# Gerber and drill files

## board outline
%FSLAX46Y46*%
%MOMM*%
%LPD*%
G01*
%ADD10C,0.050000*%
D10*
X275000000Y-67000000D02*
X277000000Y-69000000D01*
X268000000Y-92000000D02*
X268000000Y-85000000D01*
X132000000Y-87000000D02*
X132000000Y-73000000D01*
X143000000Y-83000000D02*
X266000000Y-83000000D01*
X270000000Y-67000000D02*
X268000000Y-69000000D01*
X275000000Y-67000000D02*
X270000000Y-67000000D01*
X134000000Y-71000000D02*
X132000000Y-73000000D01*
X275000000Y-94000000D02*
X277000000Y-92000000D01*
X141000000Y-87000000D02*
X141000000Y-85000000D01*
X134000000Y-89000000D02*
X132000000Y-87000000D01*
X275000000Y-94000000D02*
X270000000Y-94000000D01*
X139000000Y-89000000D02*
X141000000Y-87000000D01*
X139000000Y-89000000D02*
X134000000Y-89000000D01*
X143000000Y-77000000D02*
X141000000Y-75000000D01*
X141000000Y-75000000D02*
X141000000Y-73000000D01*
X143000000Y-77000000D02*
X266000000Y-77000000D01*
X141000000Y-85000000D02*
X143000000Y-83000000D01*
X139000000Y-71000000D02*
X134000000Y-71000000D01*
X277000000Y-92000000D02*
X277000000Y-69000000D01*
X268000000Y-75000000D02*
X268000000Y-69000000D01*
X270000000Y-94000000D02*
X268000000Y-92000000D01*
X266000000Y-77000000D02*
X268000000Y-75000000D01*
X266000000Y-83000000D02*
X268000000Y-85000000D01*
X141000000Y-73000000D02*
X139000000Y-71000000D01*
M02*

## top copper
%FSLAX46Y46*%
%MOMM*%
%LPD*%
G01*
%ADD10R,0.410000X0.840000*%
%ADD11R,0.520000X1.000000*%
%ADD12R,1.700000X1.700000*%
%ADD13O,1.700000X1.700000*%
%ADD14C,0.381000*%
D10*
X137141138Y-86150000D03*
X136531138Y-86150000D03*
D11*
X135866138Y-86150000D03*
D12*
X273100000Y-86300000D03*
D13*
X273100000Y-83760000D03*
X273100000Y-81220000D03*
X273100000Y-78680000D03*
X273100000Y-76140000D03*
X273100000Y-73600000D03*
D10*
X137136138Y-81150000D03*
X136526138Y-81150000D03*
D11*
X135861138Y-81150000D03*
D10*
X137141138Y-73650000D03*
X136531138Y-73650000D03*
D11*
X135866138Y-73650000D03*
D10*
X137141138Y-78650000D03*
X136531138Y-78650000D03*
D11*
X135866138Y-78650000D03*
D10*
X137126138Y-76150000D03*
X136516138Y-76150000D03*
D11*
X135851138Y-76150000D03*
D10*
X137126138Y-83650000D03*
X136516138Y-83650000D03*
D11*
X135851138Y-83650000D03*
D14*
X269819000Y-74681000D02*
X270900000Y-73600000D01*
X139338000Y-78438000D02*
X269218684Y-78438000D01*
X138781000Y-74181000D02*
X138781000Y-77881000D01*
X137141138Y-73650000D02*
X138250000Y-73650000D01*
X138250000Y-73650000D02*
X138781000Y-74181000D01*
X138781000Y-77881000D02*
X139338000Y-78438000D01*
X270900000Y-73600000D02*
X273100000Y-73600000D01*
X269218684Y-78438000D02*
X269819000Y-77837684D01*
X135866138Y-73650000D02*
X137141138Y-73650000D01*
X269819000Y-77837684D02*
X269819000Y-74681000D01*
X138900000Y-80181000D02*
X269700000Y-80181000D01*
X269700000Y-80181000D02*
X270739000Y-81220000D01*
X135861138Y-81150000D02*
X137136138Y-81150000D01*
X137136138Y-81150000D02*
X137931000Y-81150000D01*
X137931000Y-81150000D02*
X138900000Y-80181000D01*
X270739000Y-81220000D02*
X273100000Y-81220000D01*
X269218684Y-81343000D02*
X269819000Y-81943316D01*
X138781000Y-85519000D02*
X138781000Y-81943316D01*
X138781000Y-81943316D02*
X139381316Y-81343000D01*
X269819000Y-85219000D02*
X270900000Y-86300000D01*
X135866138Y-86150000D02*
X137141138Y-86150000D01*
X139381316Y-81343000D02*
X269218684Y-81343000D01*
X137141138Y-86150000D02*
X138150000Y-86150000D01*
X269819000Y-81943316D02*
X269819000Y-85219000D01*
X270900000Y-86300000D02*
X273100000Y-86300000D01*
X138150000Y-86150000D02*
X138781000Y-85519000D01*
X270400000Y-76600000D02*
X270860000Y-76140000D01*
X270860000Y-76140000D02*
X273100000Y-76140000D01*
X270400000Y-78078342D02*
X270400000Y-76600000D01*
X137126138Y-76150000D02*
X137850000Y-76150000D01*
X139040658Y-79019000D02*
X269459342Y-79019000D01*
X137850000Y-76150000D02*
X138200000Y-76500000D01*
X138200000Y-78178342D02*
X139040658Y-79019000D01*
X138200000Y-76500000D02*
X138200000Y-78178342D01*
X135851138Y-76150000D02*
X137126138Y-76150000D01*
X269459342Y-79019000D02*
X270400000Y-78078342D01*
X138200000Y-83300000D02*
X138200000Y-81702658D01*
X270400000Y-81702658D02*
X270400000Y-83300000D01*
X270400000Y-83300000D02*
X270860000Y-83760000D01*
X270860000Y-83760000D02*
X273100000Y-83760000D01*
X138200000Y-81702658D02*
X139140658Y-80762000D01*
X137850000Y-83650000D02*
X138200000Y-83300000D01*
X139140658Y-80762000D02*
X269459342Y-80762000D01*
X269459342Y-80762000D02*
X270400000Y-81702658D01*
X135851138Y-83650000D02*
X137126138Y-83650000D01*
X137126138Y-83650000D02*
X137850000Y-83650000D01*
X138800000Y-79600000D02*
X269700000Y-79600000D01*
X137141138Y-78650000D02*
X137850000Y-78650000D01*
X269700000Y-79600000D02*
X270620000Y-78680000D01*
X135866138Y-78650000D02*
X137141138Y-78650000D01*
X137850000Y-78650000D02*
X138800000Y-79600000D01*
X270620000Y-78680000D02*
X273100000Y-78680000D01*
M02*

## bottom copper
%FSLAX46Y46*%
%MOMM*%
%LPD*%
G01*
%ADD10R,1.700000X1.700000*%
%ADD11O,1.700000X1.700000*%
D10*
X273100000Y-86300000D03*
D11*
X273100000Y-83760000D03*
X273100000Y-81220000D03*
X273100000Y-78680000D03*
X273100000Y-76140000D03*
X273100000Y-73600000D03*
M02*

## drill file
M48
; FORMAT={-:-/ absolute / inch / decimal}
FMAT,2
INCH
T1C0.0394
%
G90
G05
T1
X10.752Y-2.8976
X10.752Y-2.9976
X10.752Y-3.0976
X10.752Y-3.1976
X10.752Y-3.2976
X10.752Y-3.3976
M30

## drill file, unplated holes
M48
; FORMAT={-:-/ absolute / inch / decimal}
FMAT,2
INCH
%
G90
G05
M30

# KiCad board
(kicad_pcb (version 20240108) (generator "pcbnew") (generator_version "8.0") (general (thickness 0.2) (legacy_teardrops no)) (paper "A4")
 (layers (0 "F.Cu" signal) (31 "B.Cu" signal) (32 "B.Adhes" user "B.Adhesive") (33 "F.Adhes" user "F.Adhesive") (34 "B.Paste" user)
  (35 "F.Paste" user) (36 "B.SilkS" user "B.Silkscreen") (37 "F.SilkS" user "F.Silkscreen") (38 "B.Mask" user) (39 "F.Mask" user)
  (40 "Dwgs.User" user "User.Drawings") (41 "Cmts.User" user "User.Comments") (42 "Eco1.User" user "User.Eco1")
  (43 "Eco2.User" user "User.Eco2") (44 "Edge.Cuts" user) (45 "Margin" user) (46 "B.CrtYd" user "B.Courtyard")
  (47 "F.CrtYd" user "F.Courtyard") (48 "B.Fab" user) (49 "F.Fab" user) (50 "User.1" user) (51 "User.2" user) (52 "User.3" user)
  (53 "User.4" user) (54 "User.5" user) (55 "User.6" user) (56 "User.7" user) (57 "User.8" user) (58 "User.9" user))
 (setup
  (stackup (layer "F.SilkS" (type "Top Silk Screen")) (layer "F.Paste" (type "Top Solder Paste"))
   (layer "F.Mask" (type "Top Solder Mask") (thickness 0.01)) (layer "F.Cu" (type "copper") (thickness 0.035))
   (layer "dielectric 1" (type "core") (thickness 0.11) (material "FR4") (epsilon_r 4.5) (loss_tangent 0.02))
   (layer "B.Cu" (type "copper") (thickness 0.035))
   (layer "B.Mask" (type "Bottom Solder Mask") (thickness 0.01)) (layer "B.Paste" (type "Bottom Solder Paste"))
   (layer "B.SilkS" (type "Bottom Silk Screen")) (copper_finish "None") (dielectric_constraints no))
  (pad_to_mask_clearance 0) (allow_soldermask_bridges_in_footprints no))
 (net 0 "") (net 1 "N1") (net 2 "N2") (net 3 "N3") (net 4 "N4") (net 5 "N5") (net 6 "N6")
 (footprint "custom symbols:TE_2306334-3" (layer "F.Cu") (at 136.446138 86.15 180)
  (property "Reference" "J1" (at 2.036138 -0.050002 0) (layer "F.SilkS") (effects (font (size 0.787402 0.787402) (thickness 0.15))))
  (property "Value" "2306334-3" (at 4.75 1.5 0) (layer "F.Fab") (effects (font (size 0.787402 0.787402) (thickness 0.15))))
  (pad "1_1" smd rect (at -0.695 0 180) (size 0.41 0.84) (layers "F.Cu" "F.Paste" "F.Mask") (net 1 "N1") (solder_mask_margin 0.102))
  (pad "1_2" smd rect (at -0.085 0 180) (size 0.41 0.84) (layers "F.Cu" "F.Paste" "F.Mask") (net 1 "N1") (solder_mask_margin 0.102))
  (pad "1_3" smd rect (at 0.58 0 180) (size 0.52 1) (layers "F.Cu" "F.Paste" "F.Mask") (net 1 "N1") (solder_mask_margin 0.102)))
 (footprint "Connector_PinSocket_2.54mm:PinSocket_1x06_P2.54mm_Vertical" (layer "F.Cu") (at 273.1 86.3 180)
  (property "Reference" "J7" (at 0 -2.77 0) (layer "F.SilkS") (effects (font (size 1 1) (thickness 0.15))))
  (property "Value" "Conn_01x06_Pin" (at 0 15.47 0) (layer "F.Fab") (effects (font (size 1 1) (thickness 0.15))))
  (pad "1" thru_hole rect (at 0 0 180) (size 1.7 1.7) (drill 1) (layers "*.Cu" "*.Mask") (remove_unused_layers no) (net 1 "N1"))
  (pad "2" thru_hole oval (at 0 2.54 180) (size 1.7 1.7) (drill 1) (layers "*.Cu" "*.Mask") (remove_unused_layers no) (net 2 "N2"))
  (pad "3" thru_hole oval (at 0 5.08 180) (size 1.7 1.7) (drill 1) (layers "*.Cu" "*.Mask") (remove_unused_layers no) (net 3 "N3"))
  (pad "4" thru_hole oval (at 0 7.62 180) (size 1.7 1.7) (drill 1) (layers "*.Cu" "*.Mask") (remove_unused_layers no) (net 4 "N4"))
  (pad "5" thru_hole oval (at 0 10.16 180) (size 1.7 1.7) (drill 1) (layers "*.Cu" "*.Mask") (remove_unused_layers no) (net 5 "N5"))
  (pad "6" thru_hole oval (at 0 12.7 180) (size 1.7 1.7) (drill 1) (layers "*.Cu" "*.Mask") (remove_unused_layers no) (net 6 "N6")))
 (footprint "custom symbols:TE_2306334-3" (layer "F.Cu") (at 136.441138 81.15 180)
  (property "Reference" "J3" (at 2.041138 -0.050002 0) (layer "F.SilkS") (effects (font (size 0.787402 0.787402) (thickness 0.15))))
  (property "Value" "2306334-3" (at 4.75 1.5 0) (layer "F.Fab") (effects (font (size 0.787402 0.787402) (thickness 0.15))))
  (pad "1_1" smd rect (at -0.695 0 180) (size 0.41 0.84) (layers "F.Cu" "F.Paste" "F.Mask") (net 3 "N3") (solder_mask_margin 0.102))
  (pad "1_2" smd rect (at -0.085 0 180) (size 0.41 0.84) (layers "F.Cu" "F.Paste" "F.Mask") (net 3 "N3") (solder_mask_margin 0.102))
  (pad "1_3" smd rect (at 0.58 0 180) (size 0.52 1) (layers "F.Cu" "F.Paste" "F.Mask") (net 3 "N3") (solder_mask_margin 0.102)))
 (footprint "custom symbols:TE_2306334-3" (layer "F.Cu") (at 136.446138 73.65 180)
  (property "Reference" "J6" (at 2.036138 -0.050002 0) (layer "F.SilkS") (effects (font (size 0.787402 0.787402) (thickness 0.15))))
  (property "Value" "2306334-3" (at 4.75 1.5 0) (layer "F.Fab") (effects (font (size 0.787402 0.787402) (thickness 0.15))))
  (pad "1_1" smd rect (at -0.695 0 180) (size 0.41 0.84) (layers "F.Cu" "F.Paste" "F.Mask") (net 6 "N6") (solder_mask_margin 0.102))
  (pad "1_2" smd rect (at -0.085 0 180) (size 0.41 0.84) (layers "F.Cu" "F.Paste" "F.Mask") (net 6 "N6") (solder_mask_margin 0.102))
  (pad "1_3" smd rect (at 0.58 0 180) (size 0.52 1) (layers "F.Cu" "F.Paste" "F.Mask") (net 6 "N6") (solder_mask_margin 0.102)))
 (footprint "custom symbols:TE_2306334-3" (layer "F.Cu") (at 136.446138 78.65 180)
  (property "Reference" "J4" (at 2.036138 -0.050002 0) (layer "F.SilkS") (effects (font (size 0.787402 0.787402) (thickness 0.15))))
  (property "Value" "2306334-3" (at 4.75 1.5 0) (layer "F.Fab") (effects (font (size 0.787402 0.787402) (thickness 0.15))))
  (pad "1_1" smd rect (at -0.695 0 180) (size 0.41 0.84) (layers "F.Cu" "F.Paste" "F.Mask") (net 4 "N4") (solder_mask_margin 0.102))
  (pad "1_2" smd rect (at -0.085 0 180) (size 0.41 0.84) (layers "F.Cu" "F.Paste" "F.Mask") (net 4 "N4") (solder_mask_margin 0.102))
  (pad "1_3" smd rect (at 0.58 0 180) (size 0.52 1) (layers "F.Cu" "F.Paste" "F.Mask") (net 4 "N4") (solder_mask_margin 0.102)))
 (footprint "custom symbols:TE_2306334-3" (layer "F.Cu") (at 136.431138 76.15 180)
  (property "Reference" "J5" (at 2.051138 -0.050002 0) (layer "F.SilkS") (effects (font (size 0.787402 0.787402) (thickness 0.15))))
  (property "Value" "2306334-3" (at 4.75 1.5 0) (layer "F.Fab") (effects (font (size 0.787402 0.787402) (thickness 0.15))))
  (pad "1_1" smd rect (at -0.695 0 180) (size 0.41 0.84) (layers "F.Cu" "F.Paste" "F.Mask") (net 5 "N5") (solder_mask_margin 0.102))
  (pad "1_2" smd rect (at -0.085 0 180) (size 0.41 0.84) (layers "F.Cu" "F.Paste" "F.Mask") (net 5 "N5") (solder_mask_margin 0.102))
  (pad "1_3" smd rect (at 0.58 0 180) (size 0.52 1) (layers "F.Cu" "F.Paste" "F.Mask") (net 5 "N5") (solder_mask_margin 0.102)))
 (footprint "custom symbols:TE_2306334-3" (layer "F.Cu") (at 136.431138 83.65 180)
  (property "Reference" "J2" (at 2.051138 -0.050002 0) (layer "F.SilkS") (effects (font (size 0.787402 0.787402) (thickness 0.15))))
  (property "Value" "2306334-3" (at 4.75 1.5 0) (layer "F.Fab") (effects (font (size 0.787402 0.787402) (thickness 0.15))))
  (pad "1_1" smd rect (at -0.695 0 180) (size 0.41 0.84) (layers "F.Cu" "F.Paste" "F.Mask") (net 2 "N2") (solder_mask_margin 0.102))
  (pad "1_2" smd rect (at -0.085 0 180) (size 0.41 0.84) (layers "F.Cu" "F.Paste" "F.Mask") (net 2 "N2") (solder_mask_margin 0.102))
  (pad "1_3" smd rect (at 0.58 0 180) (size 0.52 1) (layers "F.Cu" "F.Paste" "F.Mask") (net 2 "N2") (solder_mask_margin 0.102)))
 (gr_line (start 275 67) (end 277 69) (stroke (width 0.05) (type default)) (layer "Edge.Cuts"))
 (gr_line (start 268 92) (end 268 85) (stroke (width 0.05) (type default)) (layer "Edge.Cuts"))
 (gr_line (start 132 87) (end 132 73) (stroke (width 0.05) (type default)) (layer "Edge.Cuts"))
 (gr_line (start 143 83) (end 266 83) (stroke (width 0.05) (type default)) (layer "Edge.Cuts"))
 (gr_line (start 270 67) (end 268 69) (stroke (width 0.05) (type default)) (layer "Edge.Cuts"))
 (gr_line (start 275 67) (end 270 67) (stroke (width 0.05) (type default)) (layer "Edge.Cuts"))
 (gr_line (start 134 71) (end 132 73) (stroke (width 0.05) (type default)) (layer "Edge.Cuts"))
 (gr_line (start 275 94) (end 277 92) (stroke (width 0.05) (type default)) (layer "Edge.Cuts"))
 (gr_line (start 141 87) (end 141 85) (stroke (width 0.05) (type default)) (layer "Edge.Cuts"))
 (gr_line (start 134 89) (end 132 87) (stroke (width 0.05) (type default)) (layer "Edge.Cuts"))
 (gr_line (start 275 94) (end 270 94) (stroke (width 0.05) (type default)) (layer "Edge.Cuts"))
 (gr_line (start 139 89) (end 141 87) (stroke (width 0.05) (type default)) (layer "Edge.Cuts"))
 (gr_line (start 139 89) (end 134 89) (stroke (width 0.05) (type default)) (layer "Edge.Cuts"))
 (gr_line (start 143 77) (end 141 75) (stroke (width 0.05) (type default)) (layer "Edge.Cuts"))
 (gr_line (start 141 75) (end 141 73) (stroke (width 0.05) (type default)) (layer "Edge.Cuts"))
 (gr_line (start 143 77) (end 266 77) (stroke (width 0.05) (type default)) (layer "Edge.Cuts"))
 (gr_line (start 141 85) (end 143 83) (stroke (width 0.05) (type default)) (layer "Edge.Cuts"))
 (gr_line (start 139 71) (end 134 71) (stroke (width 0.05) (type default)) (layer "Edge.Cuts"))
 (gr_line (start 277 92) (end 277 69) (stroke (width 0.05) (type default)) (layer "Edge.Cuts"))
 (gr_line (start 268 75) (end 268 69) (stroke (width 0.05) (type default)) (layer "Edge.Cuts"))
 (gr_line (start 270 94) (end 268 92) (stroke (width 0.05) (type default)) (layer "Edge.Cuts"))
 (gr_line (start 266 77) (end 268 75) (stroke (width 0.05) (type default)) (layer "Edge.Cuts"))
 (gr_line (start 266 83) (end 268 85) (stroke (width 0.05) (type default)) (layer "Edge.Cuts"))
 (gr_line (start 141 73) (end 139 71) (stroke (width 0.05) (type default)) (layer "Edge.Cuts"))
 (segment (start 269.819 74.681) (end 270.9 73.6) (width 0.381) (layer "F.Cu") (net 6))
 (segment (start 139.338 78.438) (end 269.218684 78.438) (width 0.381) (layer "F.Cu") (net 6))
 (segment (start 138.781 74.181) (end 138.781 77.881) (width 0.381) (layer "F.Cu") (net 6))
 (segment (start 137.141138 73.65) (end 138.25 73.65) (width 0.381) (layer "F.Cu") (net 6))
 (segment (start 138.25 73.65) (end 138.781 74.181) (width 0.381) (layer "F.Cu") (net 6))
 (segment (start 138.781 77.881) (end 139.338 78.438) (width 0.381) (layer "F.Cu") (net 6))
 (segment (start 270.9 73.6) (end 273.1 73.6) (width 0.381) (layer "F.Cu") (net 6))
 (segment (start 269.218684 78.438) (end 269.819 77.837684) (width 0.381) (layer "F.Cu") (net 6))
 (segment (start 135.866138 73.65) (end 137.141138 73.65) (width 0.381) (layer "F.Cu") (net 6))
 (segment (start 269.819 77.837684) (end 269.819 74.681) (width 0.381) (layer "F.Cu") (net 6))
 (segment (start 138.9 80.181) (end 269.7 80.181) (width 0.381) (layer "F.Cu") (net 3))
 (segment (start 269.7 80.181) (end 270.739 81.22) (width 0.381) (layer "F.Cu") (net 3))
 (segment (start 135.861138 81.15) (end 137.136138 81.15) (width 0.381) (layer "F.Cu") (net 3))
 (segment (start 137.136138 81.15) (end 137.931 81.15) (width 0.381) (layer "F.Cu") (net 3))
 (segment (start 137.931 81.15) (end 138.9 80.181) (width 0.381) (layer "F.Cu") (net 3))
 (segment (start 270.739 81.22) (end 273.1 81.22) (width 0.381) (layer "F.Cu") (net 3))
 (segment (start 269.218684 81.343) (end 269.819 81.943316) (width 0.381) (layer "F.Cu") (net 1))
 (segment (start 138.781 85.519) (end 138.781 81.943316) (width 0.381) (layer "F.Cu") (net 1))
 (segment (start 138.781 81.943316) (end 139.381316 81.343) (width 0.381) (layer "F.Cu") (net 1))
 (segment (start 269.819 85.219) (end 270.9 86.3) (width 0.381) (layer "F.Cu") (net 1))
 (segment (start 135.866138 86.15) (end 137.141138 86.15) (width 0.381) (layer "F.Cu") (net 1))
 (segment (start 139.381316 81.343) (end 269.218684 81.343) (width 0.381) (layer "F.Cu") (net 1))
 (segment (start 137.141138 86.15) (end 138.15 86.15) (width 0.381) (layer "F.Cu") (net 1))
 (segment (start 269.819 81.943316) (end 269.819 85.219) (width 0.381) (layer "F.Cu") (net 1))
 (segment (start 270.9 86.3) (end 273.1 86.3) (width 0.381) (layer "F.Cu") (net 1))
 (segment (start 138.15 86.15) (end 138.781 85.519) (width 0.381) (layer "F.Cu") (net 1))
 (segment (start 270.4 76.6) (end 270.86 76.14) (width 0.381) (layer "F.Cu") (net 5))
 (segment (start 270.86 76.14) (end 273.1 76.14) (width 0.381) (layer "F.Cu") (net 5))
 (segment (start 270.4 78.078342) (end 270.4 76.6) (width 0.381) (layer "F.Cu") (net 5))
 (segment (start 137.126138 76.15) (end 137.85 76.15) (width 0.381) (layer "F.Cu") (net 5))
 (segment (start 139.040658 79.019) (end 269.459342 79.019) (width 0.381) (layer "F.Cu") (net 5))
 (segment (start 137.85 76.15) (end 138.2 76.5) (width 0.381) (layer "F.Cu") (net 5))
 (segment (start 138.2 78.178342) (end 139.040658 79.019) (width 0.381) (layer "F.Cu") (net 5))
 (segment (start 138.2 76.5) (end 138.2 78.178342) (width 0.381) (layer "F.Cu") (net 5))
 (segment (start 135.851138 76.15) (end 137.126138 76.15) (width 0.381) (layer "F.Cu") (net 5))
 (segment (start 269.459342 79.019) (end 270.4 78.078342) (width 0.381) (layer "F.Cu") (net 5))
 (segment (start 138.2 83.3) (end 138.2 81.702658) (width 0.381) (layer "F.Cu") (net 2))
 (segment (start 270.4 81.702658) (end 270.4 83.3) (width 0.381) (layer "F.Cu") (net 2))
 (segment (start 270.4 83.3) (end 270.86 83.76) (width 0.381) (layer "F.Cu") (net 2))
 (segment (start 270.86 83.76) (end 273.1 83.76) (width 0.381) (layer "F.Cu") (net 2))
 (segment (start 138.2 81.702658) (end 139.140658 80.762) (width 0.381) (layer "F.Cu") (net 2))
 (segment (start 137.85 83.65) (end 138.2 83.3) (width 0.381) (layer "F.Cu") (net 2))
 (segment (start 139.140658 80.762) (end 269.459342 80.762) (width 0.381) (layer "F.Cu") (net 2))
 (segment (start 269.459342 80.762) (end 270.4 81.702658) (width 0.381) (layer "F.Cu") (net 2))
 (segment (start 135.851138 83.65) (end 137.126138 83.65) (width 0.381) (layer "F.Cu") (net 2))
 (segment (start 137.126138 83.65) (end 137.85 83.65) (width 0.381) (layer "F.Cu") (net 2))
 (segment (start 138.8 79.6) (end 269.7 79.6) (width 0.381) (layer "F.Cu") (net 4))
 (segment (start 137.141138 78.65) (end 137.85 78.65) (width 0.381) (layer "F.Cu") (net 4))
 (segment (start 269.7 79.6) (end 270.62 78.68) (width 0.381) (layer "F.Cu") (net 4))
 (segment (start 135.866138 78.65) (end 137.141138 78.65) (width 0.381) (layer "F.Cu") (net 4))
 (segment (start 137.85 78.65) (end 138.8 79.6) (width 0.381) (layer "F.Cu") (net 4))
 (segment (start 270.62 78.68) (end 273.1 78.68) (width 0.381) (layer "F.Cu") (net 4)))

